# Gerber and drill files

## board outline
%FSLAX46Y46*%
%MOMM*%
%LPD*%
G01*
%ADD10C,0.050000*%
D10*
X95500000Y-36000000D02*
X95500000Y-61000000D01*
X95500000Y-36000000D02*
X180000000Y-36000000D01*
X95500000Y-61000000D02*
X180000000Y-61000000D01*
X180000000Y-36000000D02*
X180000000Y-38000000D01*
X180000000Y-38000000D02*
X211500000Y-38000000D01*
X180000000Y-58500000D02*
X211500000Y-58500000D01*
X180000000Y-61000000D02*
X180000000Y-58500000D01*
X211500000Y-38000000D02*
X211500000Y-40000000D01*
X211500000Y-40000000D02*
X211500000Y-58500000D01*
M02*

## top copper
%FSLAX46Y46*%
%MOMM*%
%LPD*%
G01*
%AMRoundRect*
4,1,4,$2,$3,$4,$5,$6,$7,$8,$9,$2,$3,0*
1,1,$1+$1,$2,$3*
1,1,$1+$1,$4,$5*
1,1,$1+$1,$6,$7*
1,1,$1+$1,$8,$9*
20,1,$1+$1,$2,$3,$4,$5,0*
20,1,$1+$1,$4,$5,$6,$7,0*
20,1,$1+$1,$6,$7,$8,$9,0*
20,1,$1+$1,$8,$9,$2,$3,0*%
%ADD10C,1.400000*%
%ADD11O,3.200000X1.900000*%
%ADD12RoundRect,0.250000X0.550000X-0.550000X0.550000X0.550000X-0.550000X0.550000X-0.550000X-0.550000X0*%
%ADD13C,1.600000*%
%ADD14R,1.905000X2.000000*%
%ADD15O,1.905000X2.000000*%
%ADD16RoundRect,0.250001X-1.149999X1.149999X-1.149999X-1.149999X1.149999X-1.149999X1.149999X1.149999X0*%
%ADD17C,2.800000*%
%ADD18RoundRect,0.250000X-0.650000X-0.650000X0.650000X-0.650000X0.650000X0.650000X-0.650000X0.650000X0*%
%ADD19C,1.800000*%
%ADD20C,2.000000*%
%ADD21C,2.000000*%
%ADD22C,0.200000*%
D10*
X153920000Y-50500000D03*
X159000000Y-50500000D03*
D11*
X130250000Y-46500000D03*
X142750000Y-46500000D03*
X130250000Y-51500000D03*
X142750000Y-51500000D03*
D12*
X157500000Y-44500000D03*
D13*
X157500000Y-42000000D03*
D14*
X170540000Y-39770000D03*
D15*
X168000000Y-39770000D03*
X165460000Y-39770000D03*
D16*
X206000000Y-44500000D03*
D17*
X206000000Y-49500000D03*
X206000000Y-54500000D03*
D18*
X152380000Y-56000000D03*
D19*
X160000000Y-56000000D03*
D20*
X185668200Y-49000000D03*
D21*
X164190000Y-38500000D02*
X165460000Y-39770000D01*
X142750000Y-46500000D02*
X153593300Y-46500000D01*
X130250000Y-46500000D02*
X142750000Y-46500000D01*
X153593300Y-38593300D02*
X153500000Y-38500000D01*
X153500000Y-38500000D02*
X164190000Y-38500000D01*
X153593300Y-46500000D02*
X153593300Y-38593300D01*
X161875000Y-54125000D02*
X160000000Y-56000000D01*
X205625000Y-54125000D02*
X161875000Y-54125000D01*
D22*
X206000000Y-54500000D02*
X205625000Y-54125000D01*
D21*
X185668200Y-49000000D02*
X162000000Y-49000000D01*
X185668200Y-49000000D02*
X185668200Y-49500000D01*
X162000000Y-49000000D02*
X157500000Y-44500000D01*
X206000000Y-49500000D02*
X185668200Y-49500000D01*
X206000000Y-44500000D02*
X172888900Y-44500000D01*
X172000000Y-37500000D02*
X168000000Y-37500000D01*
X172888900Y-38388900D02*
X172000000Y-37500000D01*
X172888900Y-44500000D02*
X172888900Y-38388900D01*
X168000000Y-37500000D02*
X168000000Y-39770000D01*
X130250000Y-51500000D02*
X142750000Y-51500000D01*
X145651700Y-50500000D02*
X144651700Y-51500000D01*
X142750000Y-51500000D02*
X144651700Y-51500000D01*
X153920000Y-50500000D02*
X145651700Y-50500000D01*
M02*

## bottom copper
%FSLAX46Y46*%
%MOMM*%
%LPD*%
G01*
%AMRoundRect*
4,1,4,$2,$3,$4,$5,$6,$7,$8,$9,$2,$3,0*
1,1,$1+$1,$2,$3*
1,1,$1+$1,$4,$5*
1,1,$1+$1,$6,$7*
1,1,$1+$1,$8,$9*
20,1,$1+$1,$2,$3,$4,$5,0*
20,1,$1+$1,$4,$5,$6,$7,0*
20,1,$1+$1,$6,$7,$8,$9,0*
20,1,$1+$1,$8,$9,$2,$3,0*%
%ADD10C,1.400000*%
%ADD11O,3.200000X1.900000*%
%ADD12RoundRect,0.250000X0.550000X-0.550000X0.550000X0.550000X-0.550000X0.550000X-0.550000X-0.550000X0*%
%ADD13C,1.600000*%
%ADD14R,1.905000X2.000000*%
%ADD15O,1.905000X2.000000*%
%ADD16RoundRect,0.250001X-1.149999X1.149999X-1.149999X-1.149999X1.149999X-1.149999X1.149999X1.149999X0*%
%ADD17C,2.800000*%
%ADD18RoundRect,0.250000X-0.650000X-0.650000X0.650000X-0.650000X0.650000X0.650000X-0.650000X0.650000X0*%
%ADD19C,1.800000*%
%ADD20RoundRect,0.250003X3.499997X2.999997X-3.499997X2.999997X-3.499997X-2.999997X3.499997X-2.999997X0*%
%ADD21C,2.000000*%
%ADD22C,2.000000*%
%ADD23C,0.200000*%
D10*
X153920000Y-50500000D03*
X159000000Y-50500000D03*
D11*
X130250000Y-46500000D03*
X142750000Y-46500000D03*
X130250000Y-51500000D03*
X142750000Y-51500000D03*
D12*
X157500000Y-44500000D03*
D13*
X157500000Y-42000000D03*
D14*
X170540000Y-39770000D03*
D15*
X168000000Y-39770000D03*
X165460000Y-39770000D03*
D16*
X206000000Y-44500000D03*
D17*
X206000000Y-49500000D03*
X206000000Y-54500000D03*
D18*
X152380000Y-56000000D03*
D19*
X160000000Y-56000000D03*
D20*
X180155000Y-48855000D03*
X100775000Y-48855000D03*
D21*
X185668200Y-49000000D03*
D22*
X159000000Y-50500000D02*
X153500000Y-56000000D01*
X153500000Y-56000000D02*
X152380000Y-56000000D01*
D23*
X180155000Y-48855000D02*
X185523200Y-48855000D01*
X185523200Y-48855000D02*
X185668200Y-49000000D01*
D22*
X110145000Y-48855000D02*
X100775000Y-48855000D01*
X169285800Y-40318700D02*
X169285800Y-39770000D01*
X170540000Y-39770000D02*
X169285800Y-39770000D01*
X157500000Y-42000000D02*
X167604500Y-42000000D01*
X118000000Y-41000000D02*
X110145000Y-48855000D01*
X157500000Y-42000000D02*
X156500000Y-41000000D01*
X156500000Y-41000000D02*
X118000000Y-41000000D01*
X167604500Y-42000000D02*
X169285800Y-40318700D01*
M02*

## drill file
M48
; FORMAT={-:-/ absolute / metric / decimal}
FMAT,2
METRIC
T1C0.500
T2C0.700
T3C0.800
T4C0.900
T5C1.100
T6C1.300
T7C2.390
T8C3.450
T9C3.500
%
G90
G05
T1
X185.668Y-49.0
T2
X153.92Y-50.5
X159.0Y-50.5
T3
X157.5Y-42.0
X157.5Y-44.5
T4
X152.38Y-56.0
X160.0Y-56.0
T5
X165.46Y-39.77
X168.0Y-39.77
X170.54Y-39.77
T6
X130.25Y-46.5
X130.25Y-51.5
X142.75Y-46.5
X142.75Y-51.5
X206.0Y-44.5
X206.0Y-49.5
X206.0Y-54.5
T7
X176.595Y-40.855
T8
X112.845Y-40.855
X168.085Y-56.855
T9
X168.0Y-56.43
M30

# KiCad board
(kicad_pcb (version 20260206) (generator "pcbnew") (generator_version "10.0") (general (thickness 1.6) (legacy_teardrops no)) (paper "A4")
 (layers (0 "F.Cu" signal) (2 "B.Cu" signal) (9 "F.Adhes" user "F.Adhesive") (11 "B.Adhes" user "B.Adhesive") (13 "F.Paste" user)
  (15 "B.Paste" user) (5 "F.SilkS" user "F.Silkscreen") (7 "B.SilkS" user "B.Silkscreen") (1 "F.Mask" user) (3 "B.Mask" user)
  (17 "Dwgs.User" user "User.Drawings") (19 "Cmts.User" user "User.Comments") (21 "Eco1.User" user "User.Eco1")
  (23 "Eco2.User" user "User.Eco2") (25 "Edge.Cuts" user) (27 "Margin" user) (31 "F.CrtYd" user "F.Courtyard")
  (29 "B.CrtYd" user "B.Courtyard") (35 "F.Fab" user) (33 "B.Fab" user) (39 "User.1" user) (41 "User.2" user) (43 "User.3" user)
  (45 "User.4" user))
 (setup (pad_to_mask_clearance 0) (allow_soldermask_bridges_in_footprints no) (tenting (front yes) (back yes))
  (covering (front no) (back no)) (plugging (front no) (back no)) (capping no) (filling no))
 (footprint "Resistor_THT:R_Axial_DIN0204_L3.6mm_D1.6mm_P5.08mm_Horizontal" (layer "F.Cu") (at 153.92 50.5)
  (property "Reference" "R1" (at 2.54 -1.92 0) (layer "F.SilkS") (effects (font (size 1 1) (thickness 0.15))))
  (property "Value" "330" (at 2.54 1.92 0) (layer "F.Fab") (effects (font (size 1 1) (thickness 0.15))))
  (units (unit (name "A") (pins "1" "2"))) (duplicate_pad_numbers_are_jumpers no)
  (pad "1" thru_hole circle (at 0 0) (size 1.4 1.4) (drill 0.7) (layers "*.Cu" "*.Mask") (remove_unused_layers no) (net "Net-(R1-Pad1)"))
  (pad "2" thru_hole circle (at 5.08 0) (size 1.4 1.4) (drill 0.7) (layers "*.Cu" "*.Mask") (remove_unused_layers no) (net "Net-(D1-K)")))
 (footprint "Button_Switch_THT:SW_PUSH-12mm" (layer "F.Cu") (at 130.25 46.5)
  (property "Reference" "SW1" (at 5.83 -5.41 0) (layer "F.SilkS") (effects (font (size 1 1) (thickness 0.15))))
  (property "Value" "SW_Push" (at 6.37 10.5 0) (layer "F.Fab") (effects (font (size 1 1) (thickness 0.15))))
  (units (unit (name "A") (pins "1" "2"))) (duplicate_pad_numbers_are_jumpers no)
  (pad "1" thru_hole oval (at 0 0) (size 3.2 1.9) (drill 1.3) (layers "*.Cu" "*.Mask") (remove_unused_layers no) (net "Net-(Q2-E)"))
  (pad "1" thru_hole oval (at 12.5 0) (size 3.2 1.9) (drill 1.3) (layers "*.Cu" "*.Mask") (remove_unused_layers no) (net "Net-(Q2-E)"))
  (pad "2" thru_hole oval (at 0 5) (size 3.2 1.9) (drill 1.3) (layers "*.Cu" "*.Mask") (remove_unused_layers no) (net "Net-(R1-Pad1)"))
  (pad "2" thru_hole oval (at 12.5 5) (size 3.2 1.9) (drill 1.3) (layers "*.Cu" "*.Mask") (remove_unused_layers no) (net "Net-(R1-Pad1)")))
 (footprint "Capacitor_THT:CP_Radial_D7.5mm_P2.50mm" (layer "F.Cu") (at 157.5 44.5 90)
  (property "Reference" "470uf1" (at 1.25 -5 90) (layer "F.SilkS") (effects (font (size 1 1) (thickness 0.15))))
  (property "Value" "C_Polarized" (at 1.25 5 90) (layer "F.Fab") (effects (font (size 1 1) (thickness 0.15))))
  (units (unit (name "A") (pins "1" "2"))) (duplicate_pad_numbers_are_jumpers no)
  (pad "1" thru_hole roundrect (at 0 0 90) (size 1.6 1.6) (drill 0.8) (layers "*.Cu" "*.Mask") (remove_unused_layers no)
   (roundrect_rratio 0.15625) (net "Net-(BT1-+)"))
  (pad "2" thru_hole circle (at 2.5 0 90) (size 1.6 1.6) (drill 0.8) (layers "*.Cu" "*.Mask") (remove_unused_layers no) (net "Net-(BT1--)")))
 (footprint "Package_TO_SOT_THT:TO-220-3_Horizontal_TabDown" (layer "F.Cu") (at 170.54 39.77 180)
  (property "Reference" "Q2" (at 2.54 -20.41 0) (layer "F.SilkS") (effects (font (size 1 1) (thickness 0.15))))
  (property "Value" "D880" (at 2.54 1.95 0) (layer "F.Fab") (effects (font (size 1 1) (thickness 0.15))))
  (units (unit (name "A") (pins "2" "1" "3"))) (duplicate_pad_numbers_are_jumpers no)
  (pad "" np_thru_hole circle (at 2.54 -16.66 180) (size 3.5 3.5) (drill 3.5) (layers "*.Cu" "*.Mask"))
  (pad "1" thru_hole rect (at 0 0 180) (size 1.905 2) (drill 1.1) (layers "*.Cu" "*.Mask") (remove_unused_layers no) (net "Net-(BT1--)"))
  (pad "2" thru_hole oval (at 2.54 0 180) (size 1.905 2) (drill 1.1) (layers "*.Cu" "*.Mask") (remove_unused_layers no)
   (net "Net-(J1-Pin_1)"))
  (pad "3" thru_hole oval (at 5.08 0 180) (size 1.905 2) (drill 1.1) (layers "*.Cu" "*.Mask") (remove_unused_layers no) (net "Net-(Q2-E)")))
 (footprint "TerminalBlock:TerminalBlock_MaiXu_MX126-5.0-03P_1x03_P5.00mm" (layer "F.Cu") (at 206 44.5 -90)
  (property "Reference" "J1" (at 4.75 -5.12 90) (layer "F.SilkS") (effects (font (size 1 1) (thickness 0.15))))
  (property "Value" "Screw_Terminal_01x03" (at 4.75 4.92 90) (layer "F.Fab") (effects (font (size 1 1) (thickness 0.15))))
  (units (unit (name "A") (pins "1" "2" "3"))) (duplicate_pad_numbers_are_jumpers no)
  (pad "1" thru_hole roundrect (at 0 0 270) (size 2.8 2.8) (drill 1.3) (layers "*.Cu" "*.Mask") (remove_unused_layers no)
   (roundrect_rratio 0.089286) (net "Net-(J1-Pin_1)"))
  (pad "2" thru_hole circle (at 5 0 270) (size 2.8 2.8) (drill 1.3) (layers "*.Cu" "*.Mask") (remove_unused_layers no) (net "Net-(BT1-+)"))
  (pad "3" thru_hole circle (at 10 0 270) (size 2.8 2.8) (drill 1.3) (layers "*.Cu" "*.Mask") (remove_unused_layers no) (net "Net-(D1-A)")))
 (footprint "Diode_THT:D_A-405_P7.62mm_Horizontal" (layer "F.Cu") (at 152.38 56)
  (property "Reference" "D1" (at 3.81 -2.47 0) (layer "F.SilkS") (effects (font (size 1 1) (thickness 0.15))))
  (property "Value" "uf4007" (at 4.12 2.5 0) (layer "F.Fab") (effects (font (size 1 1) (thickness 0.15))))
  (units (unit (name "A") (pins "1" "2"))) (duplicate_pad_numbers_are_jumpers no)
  (pad "1" thru_hole roundrect (at 0 0) (size 1.8 1.8) (drill 0.9) (layers "*.Cu" "*.Mask") (remove_unused_layers no)
   (roundrect_rratio 0.138889) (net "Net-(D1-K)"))
  (pad "2" thru_hole circle (at 7.62 0) (size 1.8 1.8) (drill 0.9) (layers "*.Cu" "*.Mask") (remove_unused_layers no) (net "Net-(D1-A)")))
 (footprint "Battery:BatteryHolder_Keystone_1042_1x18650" (layer "B.Cu") (at 140.465 48.855 180)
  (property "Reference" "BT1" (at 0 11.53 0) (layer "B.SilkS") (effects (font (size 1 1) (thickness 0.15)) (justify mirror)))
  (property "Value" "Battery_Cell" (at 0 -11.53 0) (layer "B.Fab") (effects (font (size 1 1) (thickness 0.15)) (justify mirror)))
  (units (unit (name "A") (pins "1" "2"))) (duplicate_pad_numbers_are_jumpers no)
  (pad "" np_thru_hole circle (at -36.13 8 180) (size 2.39 2.39) (drill 2.39) (layers "*.Cu" "*.Mask"))
  (pad "" np_thru_hole circle (at -27.62 -8 180) (size 3.45 3.45) (drill 3.45) (layers "*.Cu" "*.Mask"))
  (pad "" np_thru_hole circle (at 27.62 8 180) (size 3.45 3.45) (drill 3.45) (layers "*.Cu" "*.Mask"))
  (pad "1" smd roundrect (at -39.69 0 180) (size 7.5 6.5) (layers "B.Cu" "B.Mask" "B.Paste") (roundrect_rratio 0.038462) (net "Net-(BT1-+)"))
  (pad "2" smd roundrect (at 39.69 0 180) (size 7.5 6.5) (layers "B.Cu" "B.Mask" "B.Paste") (roundrect_rratio 0.038462) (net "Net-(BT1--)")))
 (gr_line (start 95.5 36) (end 95.5 61) (stroke (width 0.05) (type default)) (layer "Edge.Cuts"))
 (gr_line (start 95.5 36) (end 180 36) (stroke (width 0.05) (type default)) (layer "Edge.Cuts"))
 (gr_line (start 95.5 61) (end 180 61) (stroke (width 0.05) (type default)) (layer "Edge.Cuts"))
 (gr_line (start 180 36) (end 180 38) (stroke (width 0.05) (type default)) (layer "Edge.Cuts"))
 (gr_line (start 180 38) (end 211.5 38) (stroke (width 0.05) (type default)) (layer "Edge.Cuts"))
 (gr_line (start 180 58.5) (end 211.5 58.5) (stroke (width 0.05) (type default)) (layer "Edge.Cuts"))
 (gr_line (start 180 61) (end 180 58.5) (stroke (width 0.05) (type default)) (layer "Edge.Cuts"))
 (gr_line (start 211.5 38) (end 211.5 40) (stroke (width 0.05) (type default)) (layer "Edge.Cuts"))
 (gr_line (start 211.5 40) (end 211.5 58.5) (stroke (width 0.05) (type default)) (layer "Edge.Cuts"))
 (segment (start 164.19 38.5) (end 165.46 39.77) (width 2) (layer "F.Cu") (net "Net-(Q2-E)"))
 (segment (start 142.75 46.5) (end 153.5933 46.5) (width 2) (layer "F.Cu") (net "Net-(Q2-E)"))
 (segment (start 130.25 46.5) (end 142.75 46.5) (width 2) (layer "F.Cu") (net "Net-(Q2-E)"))
 (segment (start 153.5933 38.5933) (end 153.5 38.5) (width 2) (layer "F.Cu") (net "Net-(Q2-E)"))
 (segment (start 153.5 38.5) (end 164.19 38.5) (width 2) (layer "F.Cu") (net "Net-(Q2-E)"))
 (segment (start 153.5933 46.5) (end 153.5933 38.5933) (width 2) (layer "F.Cu") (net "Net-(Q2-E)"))
 (segment (start 159 50.5) (end 153.5 56) (width 2) (layer "B.Cu") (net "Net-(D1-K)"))
 (segment (start 153.5 56) (end 152.38 56) (width 2) (layer "B.Cu") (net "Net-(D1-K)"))
 (segment (start 161.875 54.125) (end 160 56) (width 2) (layer "F.Cu") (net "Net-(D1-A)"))
 (segment (start 205.625 54.125) (end 161.875 54.125) (width 2) (layer "F.Cu") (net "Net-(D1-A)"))
 (segment (start 206 54.5) (end 205.625 54.125) (width 0.2) (layer "F.Cu") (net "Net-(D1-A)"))
 (segment (start 185.6682 49) (end 162 49) (width 2) (layer "F.Cu") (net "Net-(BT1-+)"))
 (segment (start 185.6682 49) (end 185.6682 49.5) (width 2) (layer "F.Cu") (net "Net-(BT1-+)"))
 (segment (start 162 49) (end 157.5 44.5) (width 2) (layer "F.Cu") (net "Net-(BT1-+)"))
 (segment (start 206 49.5) (end 185.6682 49.5) (width 2) (layer "F.Cu") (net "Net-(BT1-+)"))
 (via (at 185.6682 49) (size 2) (drill 0.5) (layers "F.Cu" "B.Cu") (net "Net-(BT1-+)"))
 (segment (start 180.155 48.855) (end 185.5232 48.855) (width 0.2) (layer "B.Cu") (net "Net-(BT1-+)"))
 (segment (start 185.5232 48.855) (end 185.6682 49) (width 0.2) (layer "B.Cu") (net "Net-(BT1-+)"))
 (segment (start 110.145 48.855) (end 100.775 48.855) (width 2) (layer "B.Cu") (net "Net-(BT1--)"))
 (segment (start 169.2858 40.3187) (end 169.2858 39.77) (width 2) (layer "B.Cu") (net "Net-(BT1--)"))
 (segment (start 170.54 39.77) (end 169.2858 39.77) (width 2) (layer "B.Cu") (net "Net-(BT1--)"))
 (segment (start 157.5 42) (end 167.6045 42) (width 2) (layer "B.Cu") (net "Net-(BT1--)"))
 (segment (start 118 41) (end 110.145 48.855) (width 2) (layer "B.Cu") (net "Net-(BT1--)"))
 (segment (start 157.5 42) (end 156.5 41) (width 2) (layer "B.Cu") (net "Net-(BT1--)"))
 (segment (start 156.5 41) (end 118 41) (width 2) (layer "B.Cu") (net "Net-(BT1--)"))
 (segment (start 167.6045 42) (end 169.2858 40.3187) (width 2) (layer "B.Cu") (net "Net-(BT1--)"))
 (segment (start 206 44.5) (end 172.8889 44.5) (width 2) (layer "F.Cu") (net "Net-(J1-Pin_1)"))
 (segment (start 172 37.5) (end 168 37.5) (width 2) (layer "F.Cu") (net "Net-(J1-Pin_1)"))
 (segment (start 172.8889 38.3889) (end 172 37.5) (width 2) (layer "F.Cu") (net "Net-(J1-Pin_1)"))
 (segment (start 172.8889 44.5) (end 172.8889 38.3889) (width 2) (layer "F.Cu") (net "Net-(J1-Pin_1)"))
 (segment (start 168 37.5) (end 168 39.77) (width 2) (layer "F.Cu") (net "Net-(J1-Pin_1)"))
 (segment (start 130.25 51.5) (end 142.75 51.5) (width 2) (layer "F.Cu") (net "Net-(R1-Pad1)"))
 (segment (start 145.6517 50.5) (end 144.6517 51.5) (width 2) (layer "F.Cu") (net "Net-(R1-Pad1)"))
 (segment (start 142.75 51.5) (end 144.6517 51.5) (width 2) (layer "F.Cu") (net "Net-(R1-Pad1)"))
 (segment (start 153.92 50.5) (end 145.6517 50.5) (width 2) (layer "F.Cu") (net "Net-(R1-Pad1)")))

